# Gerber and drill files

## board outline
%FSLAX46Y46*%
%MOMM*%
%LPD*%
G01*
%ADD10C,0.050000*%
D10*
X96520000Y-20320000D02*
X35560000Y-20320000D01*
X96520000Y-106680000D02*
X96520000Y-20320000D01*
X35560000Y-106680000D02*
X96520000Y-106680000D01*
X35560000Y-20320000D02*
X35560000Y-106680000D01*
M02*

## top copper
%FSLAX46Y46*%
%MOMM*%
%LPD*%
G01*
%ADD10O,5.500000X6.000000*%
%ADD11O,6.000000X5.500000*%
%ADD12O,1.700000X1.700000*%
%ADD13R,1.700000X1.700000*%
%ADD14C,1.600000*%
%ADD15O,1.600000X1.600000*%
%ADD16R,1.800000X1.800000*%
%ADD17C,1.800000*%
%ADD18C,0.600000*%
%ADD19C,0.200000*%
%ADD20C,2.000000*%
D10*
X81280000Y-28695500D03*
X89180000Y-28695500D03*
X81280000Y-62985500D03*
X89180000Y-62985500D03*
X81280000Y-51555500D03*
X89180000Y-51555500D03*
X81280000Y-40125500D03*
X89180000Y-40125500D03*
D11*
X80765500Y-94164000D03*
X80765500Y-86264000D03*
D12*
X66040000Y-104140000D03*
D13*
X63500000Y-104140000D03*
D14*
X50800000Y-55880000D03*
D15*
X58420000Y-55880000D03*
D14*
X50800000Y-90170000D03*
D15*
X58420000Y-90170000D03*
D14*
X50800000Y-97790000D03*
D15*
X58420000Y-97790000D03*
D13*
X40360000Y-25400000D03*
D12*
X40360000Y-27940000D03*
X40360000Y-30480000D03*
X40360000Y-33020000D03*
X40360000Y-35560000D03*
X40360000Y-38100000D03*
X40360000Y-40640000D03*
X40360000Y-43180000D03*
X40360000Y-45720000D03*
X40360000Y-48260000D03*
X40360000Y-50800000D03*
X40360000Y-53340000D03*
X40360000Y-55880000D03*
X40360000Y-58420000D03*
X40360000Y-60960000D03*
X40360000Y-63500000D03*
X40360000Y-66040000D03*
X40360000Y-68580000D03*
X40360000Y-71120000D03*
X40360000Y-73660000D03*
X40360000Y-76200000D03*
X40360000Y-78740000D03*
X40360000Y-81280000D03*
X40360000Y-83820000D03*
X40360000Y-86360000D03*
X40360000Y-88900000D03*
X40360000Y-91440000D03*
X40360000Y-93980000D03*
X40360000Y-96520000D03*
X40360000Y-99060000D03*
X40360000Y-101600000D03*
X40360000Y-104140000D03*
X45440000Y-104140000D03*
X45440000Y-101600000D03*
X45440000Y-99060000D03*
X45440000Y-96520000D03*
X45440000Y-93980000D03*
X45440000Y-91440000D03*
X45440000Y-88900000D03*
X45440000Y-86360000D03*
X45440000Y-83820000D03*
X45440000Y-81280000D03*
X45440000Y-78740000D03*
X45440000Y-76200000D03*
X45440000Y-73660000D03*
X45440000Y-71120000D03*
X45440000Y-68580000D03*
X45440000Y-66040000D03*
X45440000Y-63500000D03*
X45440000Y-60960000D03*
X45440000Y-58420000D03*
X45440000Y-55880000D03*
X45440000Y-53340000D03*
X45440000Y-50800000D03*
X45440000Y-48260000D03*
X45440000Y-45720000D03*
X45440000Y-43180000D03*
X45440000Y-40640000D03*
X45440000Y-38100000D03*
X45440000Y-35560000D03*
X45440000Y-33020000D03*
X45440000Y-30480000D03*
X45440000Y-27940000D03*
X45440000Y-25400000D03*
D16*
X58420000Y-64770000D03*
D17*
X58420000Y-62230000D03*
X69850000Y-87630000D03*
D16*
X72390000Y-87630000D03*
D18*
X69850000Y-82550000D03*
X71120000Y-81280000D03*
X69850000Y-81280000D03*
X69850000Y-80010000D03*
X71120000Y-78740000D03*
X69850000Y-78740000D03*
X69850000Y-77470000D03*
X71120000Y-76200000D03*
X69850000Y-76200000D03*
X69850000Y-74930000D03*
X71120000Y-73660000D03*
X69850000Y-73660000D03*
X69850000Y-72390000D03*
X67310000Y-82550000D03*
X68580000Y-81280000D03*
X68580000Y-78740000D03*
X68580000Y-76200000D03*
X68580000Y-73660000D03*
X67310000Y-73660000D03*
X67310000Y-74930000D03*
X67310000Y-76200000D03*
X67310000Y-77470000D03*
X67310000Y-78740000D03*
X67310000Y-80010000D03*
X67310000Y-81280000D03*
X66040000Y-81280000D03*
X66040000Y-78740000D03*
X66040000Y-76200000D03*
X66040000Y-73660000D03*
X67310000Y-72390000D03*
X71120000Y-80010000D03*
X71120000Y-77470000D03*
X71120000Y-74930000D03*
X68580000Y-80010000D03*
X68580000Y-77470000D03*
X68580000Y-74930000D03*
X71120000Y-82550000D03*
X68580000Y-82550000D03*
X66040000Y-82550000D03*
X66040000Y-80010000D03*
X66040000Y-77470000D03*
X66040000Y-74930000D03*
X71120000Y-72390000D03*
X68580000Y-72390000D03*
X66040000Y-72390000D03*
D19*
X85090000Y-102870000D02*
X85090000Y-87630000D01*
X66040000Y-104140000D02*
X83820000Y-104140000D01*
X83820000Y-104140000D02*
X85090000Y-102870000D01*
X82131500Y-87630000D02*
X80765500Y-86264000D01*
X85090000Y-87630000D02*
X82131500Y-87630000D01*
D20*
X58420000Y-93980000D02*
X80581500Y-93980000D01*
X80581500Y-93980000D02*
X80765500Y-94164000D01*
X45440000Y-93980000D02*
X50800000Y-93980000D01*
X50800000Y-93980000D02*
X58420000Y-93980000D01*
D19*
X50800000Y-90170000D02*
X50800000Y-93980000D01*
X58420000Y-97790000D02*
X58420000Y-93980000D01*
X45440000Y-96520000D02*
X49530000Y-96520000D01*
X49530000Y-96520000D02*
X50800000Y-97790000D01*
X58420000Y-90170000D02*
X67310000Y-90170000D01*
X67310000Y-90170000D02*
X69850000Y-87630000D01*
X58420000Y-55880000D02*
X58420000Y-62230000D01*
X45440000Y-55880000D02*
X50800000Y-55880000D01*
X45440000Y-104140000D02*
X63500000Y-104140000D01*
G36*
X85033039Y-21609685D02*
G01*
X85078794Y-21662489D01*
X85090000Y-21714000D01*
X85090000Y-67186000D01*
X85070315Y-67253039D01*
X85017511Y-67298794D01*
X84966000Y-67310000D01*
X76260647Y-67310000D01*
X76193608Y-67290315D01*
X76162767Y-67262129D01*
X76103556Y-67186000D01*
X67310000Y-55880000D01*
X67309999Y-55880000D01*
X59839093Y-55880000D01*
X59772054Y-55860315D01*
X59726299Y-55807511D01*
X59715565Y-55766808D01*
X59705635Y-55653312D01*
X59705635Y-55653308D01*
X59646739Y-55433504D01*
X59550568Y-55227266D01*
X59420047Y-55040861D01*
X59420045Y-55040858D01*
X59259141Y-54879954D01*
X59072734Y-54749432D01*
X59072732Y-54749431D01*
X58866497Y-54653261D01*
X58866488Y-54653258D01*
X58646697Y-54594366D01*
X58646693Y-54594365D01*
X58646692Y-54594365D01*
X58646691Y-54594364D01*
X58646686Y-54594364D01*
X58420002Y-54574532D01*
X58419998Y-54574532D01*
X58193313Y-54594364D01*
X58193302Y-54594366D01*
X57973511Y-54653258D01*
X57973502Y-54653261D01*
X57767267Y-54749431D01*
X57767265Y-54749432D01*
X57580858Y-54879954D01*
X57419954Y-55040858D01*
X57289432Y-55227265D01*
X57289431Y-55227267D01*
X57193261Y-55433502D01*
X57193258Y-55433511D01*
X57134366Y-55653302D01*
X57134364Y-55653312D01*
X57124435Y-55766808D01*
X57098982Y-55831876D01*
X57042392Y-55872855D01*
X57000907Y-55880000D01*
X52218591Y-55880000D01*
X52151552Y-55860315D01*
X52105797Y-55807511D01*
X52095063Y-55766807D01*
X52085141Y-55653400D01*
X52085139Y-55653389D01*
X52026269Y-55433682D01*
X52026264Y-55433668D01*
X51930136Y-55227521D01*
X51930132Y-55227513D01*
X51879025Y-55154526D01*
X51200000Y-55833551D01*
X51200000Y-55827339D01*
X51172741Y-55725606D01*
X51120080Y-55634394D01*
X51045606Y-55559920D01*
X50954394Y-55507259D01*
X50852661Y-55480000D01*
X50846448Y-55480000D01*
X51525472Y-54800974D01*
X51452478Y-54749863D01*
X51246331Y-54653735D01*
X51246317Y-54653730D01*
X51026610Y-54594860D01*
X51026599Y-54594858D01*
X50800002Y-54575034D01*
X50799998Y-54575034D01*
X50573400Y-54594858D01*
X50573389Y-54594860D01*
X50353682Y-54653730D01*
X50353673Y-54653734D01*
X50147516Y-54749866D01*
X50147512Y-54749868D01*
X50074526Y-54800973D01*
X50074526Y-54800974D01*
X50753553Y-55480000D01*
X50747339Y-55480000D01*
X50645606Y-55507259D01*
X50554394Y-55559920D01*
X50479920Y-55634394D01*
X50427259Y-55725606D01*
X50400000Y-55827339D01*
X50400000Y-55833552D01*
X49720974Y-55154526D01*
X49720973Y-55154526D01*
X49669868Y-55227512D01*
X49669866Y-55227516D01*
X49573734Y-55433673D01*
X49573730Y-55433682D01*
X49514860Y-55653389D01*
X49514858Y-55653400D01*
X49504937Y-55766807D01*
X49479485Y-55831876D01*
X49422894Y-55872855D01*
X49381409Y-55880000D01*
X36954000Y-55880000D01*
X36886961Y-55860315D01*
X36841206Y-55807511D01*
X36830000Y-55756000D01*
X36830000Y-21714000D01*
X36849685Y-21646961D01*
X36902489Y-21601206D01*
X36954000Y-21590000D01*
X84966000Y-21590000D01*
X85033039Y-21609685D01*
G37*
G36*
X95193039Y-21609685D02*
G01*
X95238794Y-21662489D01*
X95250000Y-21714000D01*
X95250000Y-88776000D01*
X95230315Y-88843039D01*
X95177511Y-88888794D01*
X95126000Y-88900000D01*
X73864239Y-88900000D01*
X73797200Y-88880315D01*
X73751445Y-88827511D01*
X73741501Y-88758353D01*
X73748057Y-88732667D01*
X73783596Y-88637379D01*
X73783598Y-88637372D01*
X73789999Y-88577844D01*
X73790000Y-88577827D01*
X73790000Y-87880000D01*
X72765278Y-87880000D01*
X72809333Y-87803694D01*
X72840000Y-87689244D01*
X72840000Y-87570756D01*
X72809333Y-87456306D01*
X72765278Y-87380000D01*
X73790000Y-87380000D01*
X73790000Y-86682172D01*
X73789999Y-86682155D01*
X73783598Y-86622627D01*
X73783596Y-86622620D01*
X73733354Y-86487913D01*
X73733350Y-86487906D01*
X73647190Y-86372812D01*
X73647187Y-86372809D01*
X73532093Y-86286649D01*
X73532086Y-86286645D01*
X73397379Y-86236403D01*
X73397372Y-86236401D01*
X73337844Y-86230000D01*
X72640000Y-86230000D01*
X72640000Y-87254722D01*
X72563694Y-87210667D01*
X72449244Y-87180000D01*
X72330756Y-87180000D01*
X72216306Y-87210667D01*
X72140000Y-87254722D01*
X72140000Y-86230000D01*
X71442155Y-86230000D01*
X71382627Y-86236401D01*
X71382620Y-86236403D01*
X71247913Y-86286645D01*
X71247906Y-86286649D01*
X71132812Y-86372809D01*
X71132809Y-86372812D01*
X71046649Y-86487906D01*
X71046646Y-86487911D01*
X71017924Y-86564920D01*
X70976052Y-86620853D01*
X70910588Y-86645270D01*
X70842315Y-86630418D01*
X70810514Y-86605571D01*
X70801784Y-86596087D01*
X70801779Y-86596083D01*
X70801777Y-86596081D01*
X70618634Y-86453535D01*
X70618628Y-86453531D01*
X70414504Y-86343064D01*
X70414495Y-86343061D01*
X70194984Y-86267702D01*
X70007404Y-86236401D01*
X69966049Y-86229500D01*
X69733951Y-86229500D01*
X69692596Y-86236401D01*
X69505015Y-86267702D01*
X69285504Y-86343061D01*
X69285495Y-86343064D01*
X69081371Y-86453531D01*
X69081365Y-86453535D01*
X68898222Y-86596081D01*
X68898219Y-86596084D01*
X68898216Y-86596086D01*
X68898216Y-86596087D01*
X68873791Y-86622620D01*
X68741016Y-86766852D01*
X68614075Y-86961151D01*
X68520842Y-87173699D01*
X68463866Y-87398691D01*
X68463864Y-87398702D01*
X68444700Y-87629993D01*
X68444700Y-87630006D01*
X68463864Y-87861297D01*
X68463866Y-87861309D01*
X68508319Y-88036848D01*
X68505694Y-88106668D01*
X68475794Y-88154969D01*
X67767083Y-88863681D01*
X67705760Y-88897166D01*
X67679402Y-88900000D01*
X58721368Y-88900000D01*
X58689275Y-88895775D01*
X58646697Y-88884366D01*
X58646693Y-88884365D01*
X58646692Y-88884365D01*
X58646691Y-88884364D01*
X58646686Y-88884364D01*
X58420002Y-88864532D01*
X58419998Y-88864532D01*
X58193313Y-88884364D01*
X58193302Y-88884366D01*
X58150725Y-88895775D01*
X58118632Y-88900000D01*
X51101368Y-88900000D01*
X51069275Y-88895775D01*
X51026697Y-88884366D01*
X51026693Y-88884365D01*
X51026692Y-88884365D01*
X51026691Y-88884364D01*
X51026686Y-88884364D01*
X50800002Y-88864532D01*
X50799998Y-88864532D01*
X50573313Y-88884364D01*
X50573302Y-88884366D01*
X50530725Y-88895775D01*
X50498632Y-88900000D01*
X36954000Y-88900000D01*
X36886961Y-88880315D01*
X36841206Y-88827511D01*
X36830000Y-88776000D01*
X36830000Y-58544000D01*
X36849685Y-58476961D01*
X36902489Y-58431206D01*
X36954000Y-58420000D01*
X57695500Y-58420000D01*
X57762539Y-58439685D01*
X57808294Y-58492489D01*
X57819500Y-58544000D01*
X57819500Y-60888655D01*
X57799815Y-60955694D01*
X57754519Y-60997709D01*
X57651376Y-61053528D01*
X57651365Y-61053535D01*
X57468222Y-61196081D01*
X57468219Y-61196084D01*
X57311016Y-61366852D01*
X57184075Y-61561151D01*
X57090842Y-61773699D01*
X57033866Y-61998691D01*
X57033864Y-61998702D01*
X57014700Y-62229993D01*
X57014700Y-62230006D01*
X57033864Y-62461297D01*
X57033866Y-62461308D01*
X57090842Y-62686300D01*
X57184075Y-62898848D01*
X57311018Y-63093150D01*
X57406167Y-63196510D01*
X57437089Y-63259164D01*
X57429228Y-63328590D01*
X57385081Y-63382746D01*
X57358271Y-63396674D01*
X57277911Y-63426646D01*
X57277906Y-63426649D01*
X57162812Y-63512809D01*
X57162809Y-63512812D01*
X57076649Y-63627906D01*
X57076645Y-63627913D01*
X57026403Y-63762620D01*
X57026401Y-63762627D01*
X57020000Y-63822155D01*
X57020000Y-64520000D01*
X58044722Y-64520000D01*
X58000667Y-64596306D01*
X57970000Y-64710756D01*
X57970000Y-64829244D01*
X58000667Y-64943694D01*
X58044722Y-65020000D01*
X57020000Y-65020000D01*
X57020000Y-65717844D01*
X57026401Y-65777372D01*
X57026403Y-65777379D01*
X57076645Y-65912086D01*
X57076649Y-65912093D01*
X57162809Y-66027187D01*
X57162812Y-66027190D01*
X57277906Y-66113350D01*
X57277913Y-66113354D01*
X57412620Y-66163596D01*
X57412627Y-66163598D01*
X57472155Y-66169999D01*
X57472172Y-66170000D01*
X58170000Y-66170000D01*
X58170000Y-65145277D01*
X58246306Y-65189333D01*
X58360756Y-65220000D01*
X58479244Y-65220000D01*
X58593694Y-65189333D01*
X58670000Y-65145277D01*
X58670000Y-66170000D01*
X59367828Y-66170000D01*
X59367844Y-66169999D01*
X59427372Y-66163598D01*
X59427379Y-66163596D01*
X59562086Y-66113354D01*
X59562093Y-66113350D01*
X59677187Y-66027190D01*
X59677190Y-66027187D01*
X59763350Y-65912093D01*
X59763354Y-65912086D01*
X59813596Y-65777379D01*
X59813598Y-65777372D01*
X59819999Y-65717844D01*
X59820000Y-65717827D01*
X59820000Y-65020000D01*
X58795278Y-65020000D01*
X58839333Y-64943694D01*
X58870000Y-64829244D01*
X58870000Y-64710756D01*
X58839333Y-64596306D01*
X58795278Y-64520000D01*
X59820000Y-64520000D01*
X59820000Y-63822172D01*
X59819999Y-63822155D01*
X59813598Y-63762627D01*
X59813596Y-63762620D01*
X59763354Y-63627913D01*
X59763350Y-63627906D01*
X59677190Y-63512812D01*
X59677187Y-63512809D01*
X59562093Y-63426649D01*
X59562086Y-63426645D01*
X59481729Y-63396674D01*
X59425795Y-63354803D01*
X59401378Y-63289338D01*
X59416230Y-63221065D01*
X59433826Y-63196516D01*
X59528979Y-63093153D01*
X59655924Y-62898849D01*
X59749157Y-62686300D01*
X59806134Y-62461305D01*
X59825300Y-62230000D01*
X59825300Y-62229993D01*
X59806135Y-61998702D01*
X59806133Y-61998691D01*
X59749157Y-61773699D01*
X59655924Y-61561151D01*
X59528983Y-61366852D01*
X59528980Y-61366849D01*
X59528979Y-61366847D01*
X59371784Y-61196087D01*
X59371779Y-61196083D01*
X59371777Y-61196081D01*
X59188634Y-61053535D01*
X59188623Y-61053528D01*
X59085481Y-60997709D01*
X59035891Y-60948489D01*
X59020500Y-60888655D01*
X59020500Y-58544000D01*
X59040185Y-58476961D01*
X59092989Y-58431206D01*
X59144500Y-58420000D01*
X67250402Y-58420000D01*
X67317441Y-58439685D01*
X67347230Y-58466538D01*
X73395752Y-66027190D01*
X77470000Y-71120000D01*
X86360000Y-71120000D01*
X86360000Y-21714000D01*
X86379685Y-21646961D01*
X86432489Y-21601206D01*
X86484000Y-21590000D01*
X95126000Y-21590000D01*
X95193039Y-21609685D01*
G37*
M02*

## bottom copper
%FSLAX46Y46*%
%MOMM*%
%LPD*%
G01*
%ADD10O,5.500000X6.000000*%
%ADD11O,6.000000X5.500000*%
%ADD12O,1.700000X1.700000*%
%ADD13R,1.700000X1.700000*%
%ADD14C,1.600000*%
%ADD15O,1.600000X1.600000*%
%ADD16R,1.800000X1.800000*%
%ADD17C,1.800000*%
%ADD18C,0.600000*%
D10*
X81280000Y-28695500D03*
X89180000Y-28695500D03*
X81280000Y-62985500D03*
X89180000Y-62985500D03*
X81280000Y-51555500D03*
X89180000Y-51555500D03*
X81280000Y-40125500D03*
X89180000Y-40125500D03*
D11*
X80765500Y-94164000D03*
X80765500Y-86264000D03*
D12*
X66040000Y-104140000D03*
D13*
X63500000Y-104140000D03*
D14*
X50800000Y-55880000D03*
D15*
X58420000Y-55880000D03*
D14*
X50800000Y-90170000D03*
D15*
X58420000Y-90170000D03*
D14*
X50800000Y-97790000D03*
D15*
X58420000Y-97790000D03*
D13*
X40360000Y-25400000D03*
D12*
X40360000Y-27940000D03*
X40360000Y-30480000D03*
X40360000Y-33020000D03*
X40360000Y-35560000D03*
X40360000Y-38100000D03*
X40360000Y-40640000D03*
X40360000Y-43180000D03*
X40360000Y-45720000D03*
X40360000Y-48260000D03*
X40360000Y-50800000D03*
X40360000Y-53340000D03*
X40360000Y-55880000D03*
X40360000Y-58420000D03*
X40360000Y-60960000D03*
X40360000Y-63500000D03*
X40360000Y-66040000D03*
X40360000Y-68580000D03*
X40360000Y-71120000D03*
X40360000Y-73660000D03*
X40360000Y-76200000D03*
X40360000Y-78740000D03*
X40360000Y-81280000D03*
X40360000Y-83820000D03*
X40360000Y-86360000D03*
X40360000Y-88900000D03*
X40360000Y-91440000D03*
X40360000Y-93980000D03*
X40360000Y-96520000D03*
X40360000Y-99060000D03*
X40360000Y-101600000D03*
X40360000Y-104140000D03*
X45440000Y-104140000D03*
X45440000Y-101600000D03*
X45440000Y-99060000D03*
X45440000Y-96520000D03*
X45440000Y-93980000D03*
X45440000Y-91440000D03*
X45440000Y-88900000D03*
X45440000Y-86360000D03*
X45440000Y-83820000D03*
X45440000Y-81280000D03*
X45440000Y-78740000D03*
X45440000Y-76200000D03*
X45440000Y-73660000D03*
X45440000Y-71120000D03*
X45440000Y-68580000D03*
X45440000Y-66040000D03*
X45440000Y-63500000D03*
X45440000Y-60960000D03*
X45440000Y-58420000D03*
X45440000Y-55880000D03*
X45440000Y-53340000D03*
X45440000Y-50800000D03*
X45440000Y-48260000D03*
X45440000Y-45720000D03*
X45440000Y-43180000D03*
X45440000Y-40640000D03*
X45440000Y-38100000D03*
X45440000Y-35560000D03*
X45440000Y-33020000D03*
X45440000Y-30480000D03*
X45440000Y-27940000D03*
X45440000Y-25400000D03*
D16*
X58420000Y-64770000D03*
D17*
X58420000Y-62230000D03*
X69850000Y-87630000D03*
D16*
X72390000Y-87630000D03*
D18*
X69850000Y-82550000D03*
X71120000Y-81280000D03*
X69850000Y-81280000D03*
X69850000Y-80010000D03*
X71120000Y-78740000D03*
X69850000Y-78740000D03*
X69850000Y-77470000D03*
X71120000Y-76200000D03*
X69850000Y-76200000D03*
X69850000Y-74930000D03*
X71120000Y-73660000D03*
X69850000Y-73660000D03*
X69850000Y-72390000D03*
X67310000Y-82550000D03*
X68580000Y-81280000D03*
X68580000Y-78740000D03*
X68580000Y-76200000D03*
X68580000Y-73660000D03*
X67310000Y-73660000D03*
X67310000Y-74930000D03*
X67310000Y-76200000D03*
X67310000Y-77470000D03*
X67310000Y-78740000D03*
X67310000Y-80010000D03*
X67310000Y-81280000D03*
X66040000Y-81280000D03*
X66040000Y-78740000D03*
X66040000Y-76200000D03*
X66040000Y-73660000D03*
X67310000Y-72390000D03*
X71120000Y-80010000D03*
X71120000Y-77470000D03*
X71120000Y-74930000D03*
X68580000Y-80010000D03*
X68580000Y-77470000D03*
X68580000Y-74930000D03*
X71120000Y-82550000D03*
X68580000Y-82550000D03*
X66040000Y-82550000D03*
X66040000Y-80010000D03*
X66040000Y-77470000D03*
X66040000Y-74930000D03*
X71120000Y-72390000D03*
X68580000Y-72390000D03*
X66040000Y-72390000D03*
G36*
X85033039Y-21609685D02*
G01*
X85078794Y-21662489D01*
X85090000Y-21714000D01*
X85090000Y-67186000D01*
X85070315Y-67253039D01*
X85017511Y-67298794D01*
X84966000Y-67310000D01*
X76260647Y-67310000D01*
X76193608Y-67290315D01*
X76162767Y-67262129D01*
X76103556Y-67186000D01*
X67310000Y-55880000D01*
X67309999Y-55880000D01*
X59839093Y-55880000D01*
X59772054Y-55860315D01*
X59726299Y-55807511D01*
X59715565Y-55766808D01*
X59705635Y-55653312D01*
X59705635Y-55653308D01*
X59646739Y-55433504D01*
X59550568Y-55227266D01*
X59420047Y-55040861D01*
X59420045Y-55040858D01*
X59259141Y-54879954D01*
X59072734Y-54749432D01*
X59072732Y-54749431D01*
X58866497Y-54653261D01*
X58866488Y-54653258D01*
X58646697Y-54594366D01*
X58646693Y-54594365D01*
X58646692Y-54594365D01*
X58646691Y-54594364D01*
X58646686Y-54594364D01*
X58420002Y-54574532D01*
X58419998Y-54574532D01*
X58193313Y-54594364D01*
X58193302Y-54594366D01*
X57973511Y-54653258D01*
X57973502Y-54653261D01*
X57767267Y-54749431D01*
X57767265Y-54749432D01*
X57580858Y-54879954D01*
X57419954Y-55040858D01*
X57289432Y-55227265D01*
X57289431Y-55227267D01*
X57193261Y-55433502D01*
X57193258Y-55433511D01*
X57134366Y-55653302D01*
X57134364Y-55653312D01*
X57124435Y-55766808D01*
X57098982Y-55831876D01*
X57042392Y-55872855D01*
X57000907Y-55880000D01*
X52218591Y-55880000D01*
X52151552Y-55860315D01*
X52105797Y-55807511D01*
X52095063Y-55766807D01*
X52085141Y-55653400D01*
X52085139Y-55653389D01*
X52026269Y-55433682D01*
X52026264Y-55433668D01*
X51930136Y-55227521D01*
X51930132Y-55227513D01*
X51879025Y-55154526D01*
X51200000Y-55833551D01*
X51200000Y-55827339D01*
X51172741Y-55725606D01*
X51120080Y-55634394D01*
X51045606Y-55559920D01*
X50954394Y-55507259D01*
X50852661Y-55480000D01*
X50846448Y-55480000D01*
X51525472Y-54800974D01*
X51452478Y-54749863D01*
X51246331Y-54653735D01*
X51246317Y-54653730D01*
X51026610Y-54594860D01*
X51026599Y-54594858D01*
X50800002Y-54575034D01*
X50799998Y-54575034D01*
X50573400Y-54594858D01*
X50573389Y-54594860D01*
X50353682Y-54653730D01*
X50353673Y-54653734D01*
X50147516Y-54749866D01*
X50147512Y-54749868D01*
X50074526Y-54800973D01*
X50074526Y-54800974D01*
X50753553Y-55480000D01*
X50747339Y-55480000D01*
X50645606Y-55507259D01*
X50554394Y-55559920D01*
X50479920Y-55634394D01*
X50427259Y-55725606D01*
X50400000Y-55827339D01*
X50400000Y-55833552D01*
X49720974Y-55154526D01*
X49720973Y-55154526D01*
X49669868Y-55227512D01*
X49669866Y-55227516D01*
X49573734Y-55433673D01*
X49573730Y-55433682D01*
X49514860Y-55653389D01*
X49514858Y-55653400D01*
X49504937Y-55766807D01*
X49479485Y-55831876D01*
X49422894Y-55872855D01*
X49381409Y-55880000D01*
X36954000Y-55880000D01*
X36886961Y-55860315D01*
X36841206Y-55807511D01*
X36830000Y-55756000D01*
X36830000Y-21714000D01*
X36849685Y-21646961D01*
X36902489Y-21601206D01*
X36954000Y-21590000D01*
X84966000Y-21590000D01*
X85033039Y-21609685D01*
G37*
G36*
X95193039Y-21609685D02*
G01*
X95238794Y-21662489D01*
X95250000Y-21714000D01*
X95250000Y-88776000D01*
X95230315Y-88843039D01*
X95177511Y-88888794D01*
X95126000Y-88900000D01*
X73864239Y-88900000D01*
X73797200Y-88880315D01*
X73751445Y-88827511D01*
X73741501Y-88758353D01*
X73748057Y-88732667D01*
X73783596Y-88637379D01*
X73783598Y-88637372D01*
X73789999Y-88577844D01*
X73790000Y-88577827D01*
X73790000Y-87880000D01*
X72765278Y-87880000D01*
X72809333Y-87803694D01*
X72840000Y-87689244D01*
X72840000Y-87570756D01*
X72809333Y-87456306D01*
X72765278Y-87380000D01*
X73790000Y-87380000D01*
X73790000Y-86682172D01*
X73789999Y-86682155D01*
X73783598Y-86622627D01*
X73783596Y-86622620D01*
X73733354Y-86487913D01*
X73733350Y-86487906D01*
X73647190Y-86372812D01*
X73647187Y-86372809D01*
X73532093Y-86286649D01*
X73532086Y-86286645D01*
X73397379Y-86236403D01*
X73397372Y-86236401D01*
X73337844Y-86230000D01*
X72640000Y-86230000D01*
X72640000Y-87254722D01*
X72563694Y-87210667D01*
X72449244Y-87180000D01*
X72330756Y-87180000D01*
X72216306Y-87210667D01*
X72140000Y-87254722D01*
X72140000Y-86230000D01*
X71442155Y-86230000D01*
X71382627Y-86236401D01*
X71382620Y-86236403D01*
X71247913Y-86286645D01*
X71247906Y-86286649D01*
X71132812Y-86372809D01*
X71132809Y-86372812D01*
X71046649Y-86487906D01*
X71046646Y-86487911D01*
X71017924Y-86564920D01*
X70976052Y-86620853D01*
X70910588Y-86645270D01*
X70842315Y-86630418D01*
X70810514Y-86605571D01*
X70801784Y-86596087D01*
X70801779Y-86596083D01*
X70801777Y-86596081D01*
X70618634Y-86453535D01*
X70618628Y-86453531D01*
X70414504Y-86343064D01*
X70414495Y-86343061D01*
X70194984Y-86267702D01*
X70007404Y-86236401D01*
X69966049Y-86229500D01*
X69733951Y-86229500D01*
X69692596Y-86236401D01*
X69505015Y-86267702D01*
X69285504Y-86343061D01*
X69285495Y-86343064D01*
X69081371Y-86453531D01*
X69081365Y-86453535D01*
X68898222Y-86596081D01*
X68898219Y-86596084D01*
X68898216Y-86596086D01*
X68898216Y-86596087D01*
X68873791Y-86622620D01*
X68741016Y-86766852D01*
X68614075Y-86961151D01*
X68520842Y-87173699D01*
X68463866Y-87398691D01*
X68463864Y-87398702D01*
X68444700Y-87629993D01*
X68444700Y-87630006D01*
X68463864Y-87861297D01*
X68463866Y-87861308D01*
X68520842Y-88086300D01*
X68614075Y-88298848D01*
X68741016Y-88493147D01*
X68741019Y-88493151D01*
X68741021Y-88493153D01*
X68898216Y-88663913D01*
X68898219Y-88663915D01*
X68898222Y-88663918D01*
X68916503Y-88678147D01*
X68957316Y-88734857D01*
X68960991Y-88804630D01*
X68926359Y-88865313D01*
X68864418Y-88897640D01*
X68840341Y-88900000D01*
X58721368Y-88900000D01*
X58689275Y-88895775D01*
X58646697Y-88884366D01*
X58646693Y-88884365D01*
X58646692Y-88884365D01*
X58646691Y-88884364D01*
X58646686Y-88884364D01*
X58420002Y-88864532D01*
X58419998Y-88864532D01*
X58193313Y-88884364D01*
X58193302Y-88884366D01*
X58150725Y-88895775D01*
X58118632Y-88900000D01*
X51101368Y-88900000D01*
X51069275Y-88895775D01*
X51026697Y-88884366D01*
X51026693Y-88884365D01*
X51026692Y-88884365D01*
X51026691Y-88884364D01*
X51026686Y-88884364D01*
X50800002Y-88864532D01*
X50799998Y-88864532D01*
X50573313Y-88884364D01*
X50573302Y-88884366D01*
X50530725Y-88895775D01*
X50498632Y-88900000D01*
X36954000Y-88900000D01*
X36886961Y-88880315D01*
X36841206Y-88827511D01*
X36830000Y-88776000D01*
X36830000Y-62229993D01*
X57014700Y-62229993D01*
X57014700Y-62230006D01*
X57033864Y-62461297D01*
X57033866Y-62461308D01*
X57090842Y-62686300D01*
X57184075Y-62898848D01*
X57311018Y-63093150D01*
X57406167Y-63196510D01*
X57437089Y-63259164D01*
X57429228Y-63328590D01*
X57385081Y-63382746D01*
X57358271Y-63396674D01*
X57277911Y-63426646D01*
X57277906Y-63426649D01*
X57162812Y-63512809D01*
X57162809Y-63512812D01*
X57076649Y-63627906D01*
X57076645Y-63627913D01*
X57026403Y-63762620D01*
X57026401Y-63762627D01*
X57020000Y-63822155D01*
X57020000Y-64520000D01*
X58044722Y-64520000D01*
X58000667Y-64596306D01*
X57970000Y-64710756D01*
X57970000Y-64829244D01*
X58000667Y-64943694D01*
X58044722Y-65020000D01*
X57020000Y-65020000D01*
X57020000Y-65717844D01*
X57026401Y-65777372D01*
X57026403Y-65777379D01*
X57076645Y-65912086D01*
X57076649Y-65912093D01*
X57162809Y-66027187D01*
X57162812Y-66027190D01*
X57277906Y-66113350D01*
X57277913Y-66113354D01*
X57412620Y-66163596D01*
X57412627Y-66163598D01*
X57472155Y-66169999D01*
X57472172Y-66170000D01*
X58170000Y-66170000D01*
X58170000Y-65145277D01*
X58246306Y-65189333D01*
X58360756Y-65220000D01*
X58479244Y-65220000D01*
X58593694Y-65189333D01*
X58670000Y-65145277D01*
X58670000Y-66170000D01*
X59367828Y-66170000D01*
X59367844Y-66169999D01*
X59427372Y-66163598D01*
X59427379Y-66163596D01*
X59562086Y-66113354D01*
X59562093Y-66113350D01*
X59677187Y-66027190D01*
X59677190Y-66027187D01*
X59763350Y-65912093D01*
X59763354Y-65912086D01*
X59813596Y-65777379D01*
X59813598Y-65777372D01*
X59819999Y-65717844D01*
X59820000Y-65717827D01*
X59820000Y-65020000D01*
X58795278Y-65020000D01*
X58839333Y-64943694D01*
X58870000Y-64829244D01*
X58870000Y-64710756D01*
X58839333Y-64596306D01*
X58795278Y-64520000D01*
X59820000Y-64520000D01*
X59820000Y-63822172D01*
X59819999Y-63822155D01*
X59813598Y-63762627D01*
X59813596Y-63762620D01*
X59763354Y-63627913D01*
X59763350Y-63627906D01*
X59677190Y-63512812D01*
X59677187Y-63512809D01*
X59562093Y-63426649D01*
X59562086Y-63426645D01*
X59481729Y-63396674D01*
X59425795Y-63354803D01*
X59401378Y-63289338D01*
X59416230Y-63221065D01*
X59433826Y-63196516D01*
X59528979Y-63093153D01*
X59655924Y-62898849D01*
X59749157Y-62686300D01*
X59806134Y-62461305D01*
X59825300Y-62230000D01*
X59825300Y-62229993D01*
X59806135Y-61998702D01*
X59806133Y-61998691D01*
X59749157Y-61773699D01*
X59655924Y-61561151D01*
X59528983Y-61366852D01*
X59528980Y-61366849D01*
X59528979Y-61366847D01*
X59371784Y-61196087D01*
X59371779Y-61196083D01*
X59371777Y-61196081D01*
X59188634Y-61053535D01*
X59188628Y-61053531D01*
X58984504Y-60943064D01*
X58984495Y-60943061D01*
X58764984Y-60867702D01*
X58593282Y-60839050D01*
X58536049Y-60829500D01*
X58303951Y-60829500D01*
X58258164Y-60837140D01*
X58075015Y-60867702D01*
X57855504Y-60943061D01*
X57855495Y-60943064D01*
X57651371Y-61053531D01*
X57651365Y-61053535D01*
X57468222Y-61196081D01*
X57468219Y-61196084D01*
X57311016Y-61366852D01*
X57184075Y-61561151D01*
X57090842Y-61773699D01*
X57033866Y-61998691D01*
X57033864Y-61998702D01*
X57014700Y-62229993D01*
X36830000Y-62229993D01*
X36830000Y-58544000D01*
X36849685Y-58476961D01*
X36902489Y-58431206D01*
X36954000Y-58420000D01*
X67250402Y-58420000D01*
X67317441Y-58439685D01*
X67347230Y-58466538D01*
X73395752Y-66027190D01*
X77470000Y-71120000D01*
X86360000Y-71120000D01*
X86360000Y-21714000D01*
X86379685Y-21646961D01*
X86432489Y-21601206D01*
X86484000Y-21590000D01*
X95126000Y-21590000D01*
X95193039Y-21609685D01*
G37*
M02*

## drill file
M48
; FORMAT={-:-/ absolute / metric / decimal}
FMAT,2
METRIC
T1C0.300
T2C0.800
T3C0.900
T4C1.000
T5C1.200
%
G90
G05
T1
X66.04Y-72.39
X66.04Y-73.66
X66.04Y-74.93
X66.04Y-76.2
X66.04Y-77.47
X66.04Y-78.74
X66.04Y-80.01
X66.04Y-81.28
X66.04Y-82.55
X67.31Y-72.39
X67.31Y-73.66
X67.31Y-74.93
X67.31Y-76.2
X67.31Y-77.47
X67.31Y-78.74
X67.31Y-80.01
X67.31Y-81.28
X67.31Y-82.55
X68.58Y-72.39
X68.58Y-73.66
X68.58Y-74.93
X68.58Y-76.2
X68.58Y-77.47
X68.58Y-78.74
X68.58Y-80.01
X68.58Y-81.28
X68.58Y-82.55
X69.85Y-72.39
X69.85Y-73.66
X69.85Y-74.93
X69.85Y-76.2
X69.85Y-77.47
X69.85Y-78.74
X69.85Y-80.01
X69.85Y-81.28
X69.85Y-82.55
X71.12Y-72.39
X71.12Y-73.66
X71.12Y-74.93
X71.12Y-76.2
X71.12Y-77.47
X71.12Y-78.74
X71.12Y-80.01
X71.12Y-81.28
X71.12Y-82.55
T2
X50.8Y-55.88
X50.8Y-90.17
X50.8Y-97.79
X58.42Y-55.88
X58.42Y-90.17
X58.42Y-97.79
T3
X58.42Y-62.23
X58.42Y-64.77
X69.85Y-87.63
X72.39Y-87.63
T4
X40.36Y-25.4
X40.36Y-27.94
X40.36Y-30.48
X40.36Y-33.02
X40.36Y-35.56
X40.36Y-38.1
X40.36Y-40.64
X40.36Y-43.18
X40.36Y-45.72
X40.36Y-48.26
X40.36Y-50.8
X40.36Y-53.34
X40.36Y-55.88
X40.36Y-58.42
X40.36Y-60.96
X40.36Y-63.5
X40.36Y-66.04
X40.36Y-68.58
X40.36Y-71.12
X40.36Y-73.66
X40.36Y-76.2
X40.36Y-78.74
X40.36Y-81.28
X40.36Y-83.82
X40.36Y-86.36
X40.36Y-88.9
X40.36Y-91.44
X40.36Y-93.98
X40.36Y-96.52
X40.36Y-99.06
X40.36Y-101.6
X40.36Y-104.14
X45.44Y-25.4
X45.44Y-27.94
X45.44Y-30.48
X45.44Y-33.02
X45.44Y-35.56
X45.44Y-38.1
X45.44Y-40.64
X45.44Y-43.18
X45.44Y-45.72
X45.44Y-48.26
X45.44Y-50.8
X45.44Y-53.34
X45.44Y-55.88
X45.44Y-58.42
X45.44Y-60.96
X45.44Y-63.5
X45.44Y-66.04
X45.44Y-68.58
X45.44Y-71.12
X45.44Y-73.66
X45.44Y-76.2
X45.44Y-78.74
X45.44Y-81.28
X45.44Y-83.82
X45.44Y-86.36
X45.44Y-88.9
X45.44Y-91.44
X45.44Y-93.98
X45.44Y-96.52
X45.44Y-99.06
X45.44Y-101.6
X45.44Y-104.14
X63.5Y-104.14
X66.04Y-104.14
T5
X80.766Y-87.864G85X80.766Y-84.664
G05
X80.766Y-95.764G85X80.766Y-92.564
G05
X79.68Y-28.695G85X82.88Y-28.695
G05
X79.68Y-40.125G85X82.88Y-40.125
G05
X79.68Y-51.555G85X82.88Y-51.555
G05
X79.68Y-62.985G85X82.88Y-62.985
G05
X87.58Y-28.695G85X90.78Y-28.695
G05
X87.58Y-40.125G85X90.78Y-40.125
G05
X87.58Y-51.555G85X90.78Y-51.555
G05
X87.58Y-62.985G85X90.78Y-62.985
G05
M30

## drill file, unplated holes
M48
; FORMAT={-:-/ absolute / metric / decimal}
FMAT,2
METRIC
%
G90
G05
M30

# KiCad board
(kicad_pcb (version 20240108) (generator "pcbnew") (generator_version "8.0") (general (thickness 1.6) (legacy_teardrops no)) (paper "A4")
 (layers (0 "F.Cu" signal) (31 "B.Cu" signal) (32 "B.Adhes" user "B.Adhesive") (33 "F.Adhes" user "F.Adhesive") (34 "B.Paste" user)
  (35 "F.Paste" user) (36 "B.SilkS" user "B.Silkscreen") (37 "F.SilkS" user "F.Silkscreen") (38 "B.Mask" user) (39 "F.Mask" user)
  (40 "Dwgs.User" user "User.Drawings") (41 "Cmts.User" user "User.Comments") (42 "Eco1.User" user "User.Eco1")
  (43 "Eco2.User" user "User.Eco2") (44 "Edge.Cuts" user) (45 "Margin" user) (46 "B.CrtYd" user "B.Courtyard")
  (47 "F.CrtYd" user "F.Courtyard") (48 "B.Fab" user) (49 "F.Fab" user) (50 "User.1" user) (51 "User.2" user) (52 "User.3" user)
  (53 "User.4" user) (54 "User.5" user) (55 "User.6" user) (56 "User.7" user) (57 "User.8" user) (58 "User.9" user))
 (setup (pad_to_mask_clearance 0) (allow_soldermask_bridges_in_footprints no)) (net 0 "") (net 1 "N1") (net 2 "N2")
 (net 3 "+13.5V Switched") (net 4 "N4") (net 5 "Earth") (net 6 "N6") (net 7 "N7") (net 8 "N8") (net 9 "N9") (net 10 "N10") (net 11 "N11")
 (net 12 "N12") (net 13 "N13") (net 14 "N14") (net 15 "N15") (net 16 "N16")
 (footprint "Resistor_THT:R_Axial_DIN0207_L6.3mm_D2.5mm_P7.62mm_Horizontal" (layer "F.Cu") (at 50.8 97.79)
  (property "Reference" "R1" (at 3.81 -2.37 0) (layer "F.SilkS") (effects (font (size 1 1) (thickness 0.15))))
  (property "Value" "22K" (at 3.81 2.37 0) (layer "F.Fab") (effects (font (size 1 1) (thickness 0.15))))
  (pad "1" thru_hole circle (at 0 0) (size 1.6 1.6) (drill 0.8) (layers "*.Cu" "*.Mask") (remove_unused_layers no) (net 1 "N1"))
  (pad "2" thru_hole oval (at 7.62 0) (size 1.6 1.6) (drill 0.8) (layers "*.Cu" "*.Mask") (remove_unused_layers no) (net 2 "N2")))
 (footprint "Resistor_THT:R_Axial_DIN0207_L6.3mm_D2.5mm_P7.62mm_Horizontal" (layer "F.Cu") (at 50.8 55.88)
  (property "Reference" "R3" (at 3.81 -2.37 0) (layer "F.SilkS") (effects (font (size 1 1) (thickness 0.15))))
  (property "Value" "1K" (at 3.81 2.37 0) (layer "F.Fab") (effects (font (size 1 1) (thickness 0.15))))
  (pad "1" thru_hole circle (at 0 0) (size 1.6 1.6) (drill 0.8) (layers "*.Cu" "*.Mask") (remove_unused_layers no) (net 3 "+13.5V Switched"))
  (pad "2" thru_hole oval (at 7.62 0) (size 1.6 1.6) (drill 0.8) (layers "*.Cu" "*.Mask") (remove_unused_layers no) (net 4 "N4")))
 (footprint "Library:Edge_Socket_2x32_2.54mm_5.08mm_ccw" (layer "F.Cu") (at 45.44 25.4)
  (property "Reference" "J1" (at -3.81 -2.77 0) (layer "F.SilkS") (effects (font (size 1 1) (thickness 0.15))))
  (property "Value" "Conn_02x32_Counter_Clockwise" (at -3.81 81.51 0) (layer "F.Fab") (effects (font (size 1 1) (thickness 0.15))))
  (pad "1" thru_hole rect (at -5.08 0) (size 1.7 1.7) (drill 1) (layers "*.Cu" "*.Mask") (remove_unused_layers no) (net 3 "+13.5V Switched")
   (zone_connect 2))
  (pad "2" thru_hole oval (at -5.08 2.54) (size 1.7 1.7) (drill 1) (layers "*.Cu" "*.Mask") (remove_unused_layers no)
   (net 3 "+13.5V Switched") (zone_connect 2))
  (pad "3" thru_hole oval (at -5.08 5.08) (size 1.7 1.7) (drill 1) (layers "*.Cu" "*.Mask") (remove_unused_layers no)
   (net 3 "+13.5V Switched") (zone_connect 2))
  (pad "4" thru_hole oval (at -5.08 7.62) (size 1.7 1.7) (drill 1) (layers "*.Cu" "*.Mask") (remove_unused_layers no)
   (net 3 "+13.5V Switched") (zone_connect 2))
  (pad "5" thru_hole oval (at -5.08 10.16) (size 1.7 1.7) (drill 1) (layers "*.Cu" "*.Mask") (remove_unused_layers no)
   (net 3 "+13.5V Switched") (zone_connect 2))
  (pad "6" thru_hole oval (at -5.08 12.7) (size 1.7 1.7) (drill 1) (layers "*.Cu" "*.Mask") (remove_unused_layers no)
   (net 3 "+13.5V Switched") (zone_connect 2))
  (pad "7" thru_hole oval (at -5.08 15.24) (size 1.7 1.7) (drill 1) (layers "*.Cu" "*.Mask") (remove_unused_layers no)
   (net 3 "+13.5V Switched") (zone_connect 2))
  (pad "8" thru_hole oval (at -5.08 17.78) (size 1.7 1.7) (drill 1) (layers "*.Cu" "*.Mask") (remove_unused_layers no)
   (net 3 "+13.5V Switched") (zone_connect 2))
  (pad "9" thru_hole oval (at -5.08 20.32) (size 1.7 1.7) (drill 1) (layers "*.Cu" "*.Mask") (remove_unused_layers no)
   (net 3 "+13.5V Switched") (zone_connect 2))
  (pad "10" thru_hole oval (at -5.08 22.86) (size 1.7 1.7) (drill 1) (layers "*.Cu" "*.Mask") (remove_unused_layers no)
   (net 3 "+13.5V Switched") (zone_connect 2))
  (pad "11" thru_hole oval (at -5.08 25.4) (size 1.7 1.7) (drill 1) (layers "*.Cu" "*.Mask") (remove_unused_layers no)
   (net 3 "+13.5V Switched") (zone_connect 2))
  (pad "12" thru_hole oval (at -5.08 27.94) (size 1.7 1.7) (drill 1) (layers "*.Cu" "*.Mask") (remove_unused_layers no)
   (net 3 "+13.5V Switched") (zone_connect 2))
  (pad "13" thru_hole oval (at -5.08 30.48) (size 1.7 1.7) (drill 1) (layers "*.Cu" "*.Mask") (remove_unused_layers no)
   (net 3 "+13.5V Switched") (zone_connect 2))
  (pad "14" thru_hole oval (at -5.08 33.02) (size 1.7 1.7) (drill 1) (layers "*.Cu" "*.Mask") (remove_unused_layers no) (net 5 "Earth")
   (zone_connect 2))
  (pad "15" thru_hole oval (at -5.08 35.56) (size 1.7 1.7) (drill 1) (layers "*.Cu" "*.Mask") (remove_unused_layers no) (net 5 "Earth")
   (zone_connect 2))
  (pad "16" thru_hole oval (at -5.08 38.1) (size 1.7 1.7) (drill 1) (layers "*.Cu" "*.Mask") (remove_unused_layers no) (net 5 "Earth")
   (zone_connect 2))
  (pad "17" thru_hole oval (at -5.08 40.64) (size 1.7 1.7) (drill 1) (layers "*.Cu" "*.Mask") (remove_unused_layers no) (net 5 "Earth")
   (zone_connect 2))
  (pad "18" thru_hole oval (at -5.08 43.18) (size 1.7 1.7) (drill 1) (layers "*.Cu" "*.Mask") (remove_unused_layers no) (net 5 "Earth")
   (zone_connect 2))
  (pad "19" thru_hole oval (at -5.08 45.72) (size 1.7 1.7) (drill 1) (layers "*.Cu" "*.Mask") (remove_unused_layers no) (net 5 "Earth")
   (zone_connect 2))
  (pad "20" thru_hole oval (at -5.08 48.26) (size 1.7 1.7) (drill 1) (layers "*.Cu" "*.Mask") (remove_unused_layers no) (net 5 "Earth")
   (zone_connect 2))
  (pad "21" thru_hole oval (at -5.08 50.8) (size 1.7 1.7) (drill 1) (layers "*.Cu" "*.Mask") (remove_unused_layers no) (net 5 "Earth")
   (zone_connect 2))
  (pad "22" thru_hole oval (at -5.08 53.34) (size 1.7 1.7) (drill 1) (layers "*.Cu" "*.Mask") (remove_unused_layers no) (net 5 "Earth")
   (zone_connect 2))
  (pad "23" thru_hole oval (at -5.08 55.88) (size 1.7 1.7) (drill 1) (layers "*.Cu" "*.Mask") (remove_unused_layers no) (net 5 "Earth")
   (zone_connect 2))
  (pad "24" thru_hole oval (at -5.08 58.42) (size 1.7 1.7) (drill 1) (layers "*.Cu" "*.Mask") (remove_unused_layers no) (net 5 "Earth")
   (zone_connect 2))
  (pad "25" thru_hole oval (at -5.08 60.96) (size 1.7 1.7) (drill 1) (layers "*.Cu" "*.Mask") (remove_unused_layers no) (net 5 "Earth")
   (zone_connect 2))
  (pad "26" thru_hole oval (at -5.08 63.5) (size 1.7 1.7) (drill 1) (layers "*.Cu" "*.Mask") (remove_unused_layers no) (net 5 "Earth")
   (zone_connect 2))
  (pad "27" thru_hole oval (at -5.08 66.04) (size 1.7 1.7) (drill 1) (layers "*.Cu" "*.Mask") (remove_unused_layers no) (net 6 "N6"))
  (pad "28" thru_hole oval (at -5.08 68.58) (size 1.7 1.7) (drill 1) (layers "*.Cu" "*.Mask") (remove_unused_layers no) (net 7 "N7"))
  (pad "29" thru_hole oval (at -5.08 71.12) (size 1.7 1.7) (drill 1) (layers "*.Cu" "*.Mask") (remove_unused_layers no) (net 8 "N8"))
  (pad "30" thru_hole oval (at -5.08 73.66) (size 1.7 1.7) (drill 1) (layers "*.Cu" "*.Mask") (remove_unused_layers no) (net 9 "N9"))
  (pad "31" thru_hole oval (at -5.08 76.2) (size 1.7 1.7) (drill 1) (layers "*.Cu" "*.Mask") (remove_unused_layers no) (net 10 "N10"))
  (pad "32" thru_hole oval (at -5.08 78.74) (size 1.7 1.7) (drill 1) (layers "*.Cu" "*.Mask") (remove_unused_layers no) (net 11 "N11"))
  (pad "33" thru_hole oval (at 0 78.74) (size 1.7 1.7) (drill 1) (layers "*.Cu" "*.Mask") (remove_unused_layers no) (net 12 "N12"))
  (pad "34" thru_hole oval (at 0 76.2) (size 1.7 1.7) (drill 1) (layers "*.Cu" "*.Mask") (remove_unused_layers no) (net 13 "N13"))
  (pad "35" thru_hole oval (at 0 73.66) (size 1.7 1.7) (drill 1) (layers "*.Cu" "*.Mask") (remove_unused_layers no) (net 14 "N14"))
  (pad "36" thru_hole oval (at 0 71.12) (size 1.7 1.7) (drill 1) (layers "*.Cu" "*.Mask") (remove_unused_layers no) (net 1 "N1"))
  (pad "37" thru_hole oval (at 0 68.58) (size 1.7 1.7) (drill 1) (layers "*.Cu" "*.Mask") (remove_unused_layers no) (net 2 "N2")
   (zone_connect 2))
  (pad "38" thru_hole oval (at 0 66.04) (size 1.7 1.7) (drill 1) (layers "*.Cu" "*.Mask") (remove_unused_layers no) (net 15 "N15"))
  (pad "39" thru_hole oval (at 0 63.5) (size 1.7 1.7) (drill 1) (layers "*.Cu" "*.Mask") (remove_unused_layers no) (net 5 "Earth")
   (zone_connect 2))
  (pad "40" thru_hole oval (at 0 60.96) (size 1.7 1.7) (drill 1) (layers "*.Cu" "*.Mask") (remove_unused_layers no) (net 5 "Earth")
   (zone_connect 2))
  (pad "41" thru_hole oval (at 0 58.42) (size 1.7 1.7) (drill 1) (layers "*.Cu" "*.Mask") (remove_unused_layers no) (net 5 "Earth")
   (zone_connect 2))
  (pad "42" thru_hole oval (at 0 55.88) (size 1.7 1.7) (drill 1) (layers "*.Cu" "*.Mask") (remove_unused_layers no) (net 5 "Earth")
   (zone_connect 2))
  (pad "43" thru_hole oval (at 0 53.34) (size 1.7 1.7) (drill 1) (layers "*.Cu" "*.Mask") (remove_unused_layers no) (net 5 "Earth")
   (zone_connect 2))
  (pad "44" thru_hole oval (at 0 50.8) (size 1.7 1.7) (drill 1) (layers "*.Cu" "*.Mask") (remove_unused_layers no) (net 5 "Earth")
   (zone_connect 2))
  (pad "45" thru_hole oval (at 0 48.26) (size 1.7 1.7) (drill 1) (layers "*.Cu" "*.Mask") (remove_unused_layers no) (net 5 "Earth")
   (zone_connect 2))
  (pad "46" thru_hole oval (at 0 45.72) (size 1.7 1.7) (drill 1) (layers "*.Cu" "*.Mask") (remove_unused_layers no) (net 5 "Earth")
   (zone_connect 2))
  (pad "47" thru_hole oval (at 0 43.18) (size 1.7 1.7) (drill 1) (layers "*.Cu" "*.Mask") (remove_unused_layers no) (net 5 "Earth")
   (zone_connect 2))
  (pad "48" thru_hole oval (at 0 40.64) (size 1.7 1.7) (drill 1) (layers "*.Cu" "*.Mask") (remove_unused_layers no) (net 5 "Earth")
   (zone_connect 2))
  (pad "49" thru_hole oval (at 0 38.1) (size 1.7 1.7) (drill 1) (layers "*.Cu" "*.Mask") (remove_unused_layers no) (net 5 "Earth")
   (zone_connect 2))
  (pad "50" thru_hole oval (at 0 35.56) (size 1.7 1.7) (drill 1) (layers "*.Cu" "*.Mask") (remove_unused_layers no) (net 5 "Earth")
   (zone_connect 2))
  (pad "51" thru_hole oval (at 0 33.02) (size 1.7 1.7) (drill 1) (layers "*.Cu" "*.Mask") (remove_unused_layers no) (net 5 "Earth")
   (zone_connect 2))
  (pad "52" thru_hole oval (at 0 30.48) (size 1.7 1.7) (drill 1) (layers "*.Cu" "*.Mask") (remove_unused_layers no)
   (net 3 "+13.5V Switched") (zone_connect 2))
  (pad "53" thru_hole oval (at 0 27.94) (size 1.7 1.7) (drill 1) (layers "*.Cu" "*.Mask") (remove_unused_layers no)
   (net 3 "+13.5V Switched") (zone_connect 2))
  (pad "54" thru_hole oval (at 0 25.4) (size 1.7 1.7) (drill 1) (layers "*.Cu" "*.Mask") (remove_unused_layers no) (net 3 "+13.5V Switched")
   (zone_connect 2))
  (pad "55" thru_hole oval (at 0 22.86) (size 1.7 1.7) (drill 1) (layers "*.Cu" "*.Mask") (remove_unused_layers no)
   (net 3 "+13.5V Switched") (zone_connect 2))
  (pad "56" thru_hole oval (at 0 20.32) (size 1.7 1.7) (drill 1) (layers "*.Cu" "*.Mask") (remove_unused_layers no)
   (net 3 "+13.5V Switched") (zone_connect 2))
  (pad "57" thru_hole oval (at 0 17.78) (size 1.7 1.7) (drill 1) (layers "*.Cu" "*.Mask") (remove_unused_layers no)
   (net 3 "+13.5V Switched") (zone_connect 2))
  (pad "58" thru_hole oval (at 0 15.24) (size 1.7 1.7) (drill 1) (layers "*.Cu" "*.Mask") (remove_unused_layers no)
   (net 3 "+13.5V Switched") (zone_connect 2))
  (pad "59" thru_hole oval (at 0 12.7) (size 1.7 1.7) (drill 1) (layers "*.Cu" "*.Mask") (remove_unused_layers no) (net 3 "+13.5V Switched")
   (zone_connect 2))
  (pad "60" thru_hole oval (at 0 10.16) (size 1.7 1.7) (drill 1) (layers "*.Cu" "*.Mask") (remove_unused_layers no)
   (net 3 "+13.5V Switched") (zone_connect 2))
  (pad "61" thru_hole oval (at 0 7.62) (size 1.7 1.7) (drill 1) (layers "*.Cu" "*.Mask") (remove_unused_layers no) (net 3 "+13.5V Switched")
   (zone_connect 2))
  (pad "62" thru_hole oval (at 0 5.08) (size 1.7 1.7) (drill 1) (layers "*.Cu" "*.Mask") (remove_unused_layers no) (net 3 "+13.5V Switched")
   (zone_connect 2))
  (pad "63" thru_hole oval (at 0 2.54) (size 1.7 1.7) (drill 1) (layers "*.Cu" "*.Mask") (remove_unused_layers no) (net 3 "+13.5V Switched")
   (zone_connect 2))
  (pad "64" thru_hole oval (at 0 0) (size 1.7 1.7) (drill 1) (layers "*.Cu" "*.Mask") (remove_unused_layers no) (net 3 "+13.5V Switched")
   (zone_connect 2)))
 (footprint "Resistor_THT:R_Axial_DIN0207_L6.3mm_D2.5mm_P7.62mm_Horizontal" (layer "F.Cu") (at 50.8 90.17)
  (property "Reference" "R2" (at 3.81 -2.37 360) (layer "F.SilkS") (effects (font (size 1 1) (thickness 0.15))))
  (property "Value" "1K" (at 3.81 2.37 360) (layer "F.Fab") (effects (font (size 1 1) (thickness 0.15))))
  (pad "1" thru_hole circle (at 0 0) (size 1.6 1.6) (drill 0.8) (layers "*.Cu" "*.Mask") (remove_unused_layers no) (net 2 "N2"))
  (pad "2" thru_hole oval (at 7.62 0) (size 1.6 1.6) (drill 0.8) (layers "*.Cu" "*.Mask") (remove_unused_layers no) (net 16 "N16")))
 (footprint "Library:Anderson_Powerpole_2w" (layer "B.Cu") (at 81.28 51.5555)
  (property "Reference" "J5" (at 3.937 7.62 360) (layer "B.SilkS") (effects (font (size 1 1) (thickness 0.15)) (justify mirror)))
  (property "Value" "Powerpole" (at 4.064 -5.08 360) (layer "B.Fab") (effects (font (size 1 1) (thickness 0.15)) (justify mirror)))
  (pad "1" thru_hole oval (at 0 0) (size 5.5 6) (drill oval 4.4 1.2) (layers "*.Cu" "*.Mask") (remove_unused_layers no)
   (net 3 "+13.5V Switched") (zone_connect 2))
  (pad "2" thru_hole oval (at 7.9 0) (size 5.5 6) (drill oval 4.4 1.2) (layers "*.Cu" "*.Mask") (remove_unused_layers no) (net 5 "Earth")
   (zone_connect 2)))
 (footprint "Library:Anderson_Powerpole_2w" (layer "B.Cu") (at 80.7655 94.164 90)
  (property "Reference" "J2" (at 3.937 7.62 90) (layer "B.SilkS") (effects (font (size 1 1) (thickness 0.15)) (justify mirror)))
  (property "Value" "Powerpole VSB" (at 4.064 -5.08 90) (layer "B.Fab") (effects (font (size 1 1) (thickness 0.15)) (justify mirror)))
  (pad "1" thru_hole oval (at 0 0 90) (size 5.5 6) (drill oval 4.4 1.2) (layers "*.Cu" "*.Mask") (remove_unused_layers no) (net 2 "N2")
   (zone_connect 2))
  (pad "2" thru_hole oval (at 7.9 0 90) (size 5.5 6) (drill oval 4.4 1.2) (layers "*.Cu" "*.Mask") (remove_unused_layers no) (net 5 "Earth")
   (zone_connect 2)))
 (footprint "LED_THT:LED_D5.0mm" (layer "B.Cu") (at 58.42 64.77 90)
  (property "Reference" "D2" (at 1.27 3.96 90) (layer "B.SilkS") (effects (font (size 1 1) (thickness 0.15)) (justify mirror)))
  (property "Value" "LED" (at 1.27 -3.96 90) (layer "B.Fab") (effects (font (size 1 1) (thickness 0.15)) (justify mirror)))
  (pad "1" thru_hole rect (at 0 0 90) (size 1.8 1.8) (drill 0.9) (layers "*.Cu" "*.Mask") (remove_unused_layers no) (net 5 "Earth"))
  (pad "2" thru_hole circle (at 2.54 0 90) (size 1.8 1.8) (drill 0.9) (layers "*.Cu" "*.Mask") (remove_unused_layers no) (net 4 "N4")))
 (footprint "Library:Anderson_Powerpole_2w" (layer "B.Cu") (at 81.28 62.9855)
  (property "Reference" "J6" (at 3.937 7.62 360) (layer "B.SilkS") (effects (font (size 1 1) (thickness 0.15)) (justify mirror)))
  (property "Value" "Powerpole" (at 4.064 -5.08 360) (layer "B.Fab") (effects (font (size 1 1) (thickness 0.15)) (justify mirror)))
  (pad "1" thru_hole oval (at 0 0) (size 5.5 6) (drill oval 4.4 1.2) (layers "*.Cu" "*.Mask") (remove_unused_layers no)
   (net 3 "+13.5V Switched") (zone_connect 2))
  (pad "2" thru_hole oval (at 7.9 0) (size 5.5 6) (drill oval 4.4 1.2) (layers "*.Cu" "*.Mask") (remove_unused_layers no) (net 5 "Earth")
   (zone_connect 2)))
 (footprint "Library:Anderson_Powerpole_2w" (layer "B.Cu") (at 81.28 28.6955)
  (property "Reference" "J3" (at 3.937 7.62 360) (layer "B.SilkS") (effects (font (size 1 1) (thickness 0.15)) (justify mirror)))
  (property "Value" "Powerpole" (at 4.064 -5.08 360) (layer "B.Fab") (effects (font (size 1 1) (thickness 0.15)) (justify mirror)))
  (pad "1" thru_hole oval (at 0 0) (size 5.5 6) (drill oval 4.4 1.2) (layers "*.Cu" "*.Mask") (remove_unused_layers no)
   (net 3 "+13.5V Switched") (zone_connect 2))
  (pad "2" thru_hole oval (at 7.9 0) (size 5.5 6) (drill oval 4.4 1.2) (layers "*.Cu" "*.Mask") (remove_unused_layers no) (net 5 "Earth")
   (zone_connect 2)))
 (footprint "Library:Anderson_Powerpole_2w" (layer "B.Cu") (at 81.28 40.1255)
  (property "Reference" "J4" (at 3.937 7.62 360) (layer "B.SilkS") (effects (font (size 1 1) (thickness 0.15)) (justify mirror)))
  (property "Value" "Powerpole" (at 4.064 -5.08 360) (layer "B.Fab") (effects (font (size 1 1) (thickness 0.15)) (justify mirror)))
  (pad "1" thru_hole oval (at 0 0) (size 5.5 6) (drill oval 4.4 1.2) (layers "*.Cu" "*.Mask") (remove_unused_layers no)
   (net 3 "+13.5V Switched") (zone_connect 2))
  (pad "2" thru_hole oval (at 7.9 0) (size 5.5 6) (drill oval 4.4 1.2) (layers "*.Cu" "*.Mask") (remove_unused_layers no) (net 5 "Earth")
   (zone_connect 2)))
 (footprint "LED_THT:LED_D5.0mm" (layer "B.Cu") (at 72.39 87.63 180)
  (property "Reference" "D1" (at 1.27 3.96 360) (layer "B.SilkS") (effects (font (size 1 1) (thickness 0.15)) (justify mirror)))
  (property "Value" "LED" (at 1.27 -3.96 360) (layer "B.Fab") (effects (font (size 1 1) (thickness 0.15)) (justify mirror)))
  (pad "1" thru_hole rect (at 0 0 180) (size 1.8 1.8) (drill 0.9) (layers "*.Cu" "*.Mask") (remove_unused_layers no) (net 5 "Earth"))
  (pad "2" thru_hole circle (at 2.54 0 180) (size 1.8 1.8) (drill 0.9) (layers "*.Cu" "*.Mask") (remove_unused_layers no) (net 16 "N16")))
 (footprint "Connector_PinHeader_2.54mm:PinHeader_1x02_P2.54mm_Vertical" (layer "B.Cu") (at 63.5 104.14 -90)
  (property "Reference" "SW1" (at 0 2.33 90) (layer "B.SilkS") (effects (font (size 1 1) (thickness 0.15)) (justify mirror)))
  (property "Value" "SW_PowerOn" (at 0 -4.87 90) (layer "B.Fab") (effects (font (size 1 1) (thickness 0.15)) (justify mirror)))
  (pad "1" thru_hole rect (at 0 0 270) (size 1.7 1.7) (drill 1) (layers "*.Cu" "*.Mask") (remove_unused_layers no) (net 12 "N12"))
  (pad "2" thru_hole oval (at 0 -2.54 270) (size 1.7 1.7) (drill 1) (layers "*.Cu" "*.Mask") (remove_unused_layers no) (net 5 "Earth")))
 (gr_line (start 96.52 106.68) (end 96.52 20.32) (stroke (width 0.05) (type default)) (layer "Edge.Cuts"))
 (gr_line (start 35.56 20.32) (end 35.56 106.68) (stroke (width 0.05) (type default)) (layer "Edge.Cuts"))
 (gr_line (start 35.56 106.68) (end 96.52 106.68) (stroke (width 0.05) (type default)) (layer "Edge.Cuts"))
 (gr_line (start 96.52 20.32) (end 35.56 20.32) (stroke (width 0.05) (type default)) (layer "Edge.Cuts"))
 (segment (start 85.09 87.63) (end 82.1315 87.63) (width 0.2) (layer "F.Cu") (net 5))
 (segment (start 82.1315 87.63) (end 80.7655 86.264) (width 0.2) (layer "F.Cu") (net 5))
 (segment (start 85.09 102.87) (end 85.09 87.63) (width 0.2) (layer "F.Cu") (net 5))
 (segment (start 66.04 104.14) (end 83.82 104.14) (width 0.2) (layer "F.Cu") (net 5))
 (segment (start 83.82 104.14) (end 85.09 102.87) (width 0.2) (layer "F.Cu") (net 5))
 (via (at 67.31 76.2) (size 0.6) (drill 0.3) (layers "F.Cu" "B.Cu") (free yes) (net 5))
 (via (at 66.04 77.47) (size 0.6) (drill 0.3) (layers "F.Cu" "B.Cu") (free yes) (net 5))
 (via (at 68.58 73.66) (size 0.6) (drill 0.3) (layers "F.Cu" "B.Cu") (free yes) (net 5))
 (via (at 71.12 81.28) (size 0.6) (drill 0.3) (layers "F.Cu" "B.Cu") (free yes) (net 5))
 (via (at 68.58 74.93) (size 0.6) (drill 0.3) (layers "F.Cu" "B.Cu") (free yes) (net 5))
 (via (at 71.12 78.74) (size 0.6) (drill 0.3) (layers "F.Cu" "B.Cu") (free yes) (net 5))
 (via (at 68.58 78.74) (size 0.6) (drill 0.3) (layers "F.Cu" "B.Cu") (free yes) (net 5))
 (via (at 71.12 80.01) (size 0.6) (drill 0.3) (layers "F.Cu" "B.Cu") (free yes) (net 5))
 (via (at 71.12 77.47) (size 0.6) (drill 0.3) (layers "F.Cu" "B.Cu") (free yes) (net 5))
 (via (at 71.12 74.93) (size 0.6) (drill 0.3) (layers "F.Cu" "B.Cu") (free yes) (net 5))
 (via (at 66.04 73.66) (size 0.6) (drill 0.3) (layers "F.Cu" "B.Cu") (free yes) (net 5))
 (via (at 68.58 82.55) (size 0.6) (drill 0.3) (layers "F.Cu" "B.Cu") (free yes) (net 5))
 (via (at 69.85 76.2) (size 0.6) (drill 0.3) (layers "F.Cu" "B.Cu") (free yes) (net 5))
 (via (at 69.85 73.66) (size 0.6) (drill 0.3) (layers "F.Cu" "B.Cu") (free yes) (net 5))
 (via (at 67.31 72.39) (size 0.6) (drill 0.3) (layers "F.Cu" "B.Cu") (free yes) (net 5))
 (via (at 69.85 82.55) (size 0.6) (drill 0.3) (layers "F.Cu" "B.Cu") (free yes) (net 5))
 (via (at 68.58 81.28) (size 0.6) (drill 0.3) (layers "F.Cu" "B.Cu") (free yes) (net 5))
 (via (at 69.85 80.01) (size 0.6) (drill 0.3) (layers "F.Cu" "B.Cu") (free yes) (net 5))
 (via (at 66.04 82.55) (size 0.6) (drill 0.3) (layers "F.Cu" "B.Cu") (free yes) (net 5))
 (via (at 67.31 78.74) (size 0.6) (drill 0.3) (layers "F.Cu" "B.Cu") (free yes) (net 5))
 (via (at 69.85 78.74) (size 0.6) (drill 0.3) (layers "F.Cu" "B.Cu") (free yes) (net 5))
 (via (at 69.85 77.47) (size 0.6) (drill 0.3) (layers "F.Cu" "B.Cu") (free yes) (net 5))
 (via (at 66.04 74.93) (size 0.6) (drill 0.3) (layers "F.Cu" "B.Cu") (free yes) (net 5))
 (via (at 68.58 77.47) (size 0.6) (drill 0.3) (layers "F.Cu" "B.Cu") (free yes) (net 5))
 (via (at 69.85 81.28) (size 0.6) (drill 0.3) (layers "F.Cu" "B.Cu") (free yes) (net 5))
 (via (at 67.31 77.47) (size 0.6) (drill 0.3) (layers "F.Cu" "B.Cu") (free yes) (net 5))
 (via (at 67.31 73.66) (size 0.6) (drill 0.3) (layers "F.Cu" "B.Cu") (free yes) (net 5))
 (via (at 69.85 72.39) (size 0.6) (drill 0.3) (layers "F.Cu" "B.Cu") (free yes) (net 5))
 (via (at 71.12 82.55) (size 0.6) (drill 0.3) (layers "F.Cu" "B.Cu") (free yes) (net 5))
 (via (at 71.12 72.39) (size 0.6) (drill 0.3) (layers "F.Cu" "B.Cu") (free yes) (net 5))
 (via (at 68.58 72.39) (size 0.6) (drill 0.3) (layers "F.Cu" "B.Cu") (free yes) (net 5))
 (via (at 66.04 76.2) (size 0.6) (drill 0.3) (layers "F.Cu" "B.Cu") (free yes) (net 5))
 (via (at 66.04 78.74) (size 0.6) (drill 0.3) (layers "F.Cu" "B.Cu") (free yes) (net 5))
 (via (at 71.12 76.2) (size 0.6) (drill 0.3) (layers "F.Cu" "B.Cu") (free yes) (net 5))
 (via (at 67.31 80.01) (size 0.6) (drill 0.3) (layers "F.Cu" "B.Cu") (free yes) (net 5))
 (via (at 68.58 80.01) (size 0.6) (drill 0.3) (layers "F.Cu" "B.Cu") (free yes) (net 5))
 (via (at 68.58 76.2) (size 0.6) (drill 0.3) (layers "F.Cu" "B.Cu") (free yes) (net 5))
 (via (at 67.31 81.28) (size 0.6) (drill 0.3) (layers "F.Cu" "B.Cu") (free yes) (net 5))
 (via (at 67.31 82.55) (size 0.6) (drill 0.3) (layers "F.Cu" "B.Cu") (free yes) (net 5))
 (via (at 66.04 81.28) (size 0.6) (drill 0.3) (layers "F.Cu" "B.Cu") (free yes) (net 5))
 (via (at 69.85 74.93) (size 0.6) (drill 0.3) (layers "F.Cu" "B.Cu") (free yes) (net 5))
 (via (at 67.31 74.93) (size 0.6) (drill 0.3) (layers "F.Cu" "B.Cu") (free yes) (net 5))
 (via (at 71.12 73.66) (size 0.6) (drill 0.3) (layers "F.Cu" "B.Cu") (free yes) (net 5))
 (via (at 66.04 72.39) (size 0.6) (drill 0.3) (layers "F.Cu" "B.Cu") (free yes) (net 5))
 (via (at 66.04 80.01) (size 0.6) (drill 0.3) (layers "F.Cu" "B.Cu") (free yes) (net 5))
 (segment (start 58.42 90.17) (end 67.31 90.17) (width 0.2) (layer "F.Cu") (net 16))
 (segment (start 67.31 90.17) (end 69.85 87.63) (width 0.2) (layer "F.Cu") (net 16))
 (segment (start 58.42 55.88) (end 58.42 62.23) (width 0.2) (layer "F.Cu") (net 4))
 (segment (start 45.44 55.88) (end 50.8 55.88) (width 0.2) (layer "F.Cu") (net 3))
 (segment (start 45.44 96.52) (end 49.53 96.52) (width 0.2) (layer "F.Cu") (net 1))
 (segment (start 49.53 96.52) (end 50.8 97.79) (width 0.2) (layer "F.Cu") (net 1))
 (segment (start 45.44 104.14) (end 63.5 104.14) (width 0.2) (layer "F.Cu") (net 12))
 (segment (start 45.44 93.98) (end 50.8 93.98) (width 2) (layer "F.Cu") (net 2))
 (segment (start 58.42 93.98) (end 80.5815 93.98) (width 2) (layer "F.Cu") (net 2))
 (segment (start 50.8 93.98) (end 58.42 93.98) (width 2) (layer "F.Cu") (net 2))
 (segment (start 80.5815 93.98) (end 80.7655 94.164) (width 2) (layer "F.Cu") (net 2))
 (segment (start 58.42 97.79) (end 58.42 93.98) (width 0.2) (layer "F.Cu") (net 2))
 (segment (start 50.8 90.17) (end 50.8 93.98) (width 0.2) (layer "F.Cu") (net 2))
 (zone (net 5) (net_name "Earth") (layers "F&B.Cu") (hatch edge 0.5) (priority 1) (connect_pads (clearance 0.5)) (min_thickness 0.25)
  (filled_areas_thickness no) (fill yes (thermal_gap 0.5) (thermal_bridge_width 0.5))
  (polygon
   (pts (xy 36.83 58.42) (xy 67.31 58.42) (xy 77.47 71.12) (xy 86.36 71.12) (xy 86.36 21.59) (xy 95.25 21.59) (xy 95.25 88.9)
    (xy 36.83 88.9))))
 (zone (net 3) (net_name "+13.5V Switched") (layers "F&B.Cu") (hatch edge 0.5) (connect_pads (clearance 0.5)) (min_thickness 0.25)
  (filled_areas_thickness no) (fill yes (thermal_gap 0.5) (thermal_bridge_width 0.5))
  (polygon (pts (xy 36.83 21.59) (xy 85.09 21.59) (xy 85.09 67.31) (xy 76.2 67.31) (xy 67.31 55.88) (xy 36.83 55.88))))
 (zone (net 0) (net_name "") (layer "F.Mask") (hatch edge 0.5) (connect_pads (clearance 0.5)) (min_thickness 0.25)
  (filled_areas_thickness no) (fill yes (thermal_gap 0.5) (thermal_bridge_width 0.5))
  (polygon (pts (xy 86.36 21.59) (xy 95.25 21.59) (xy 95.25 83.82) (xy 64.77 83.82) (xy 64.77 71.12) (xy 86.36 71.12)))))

